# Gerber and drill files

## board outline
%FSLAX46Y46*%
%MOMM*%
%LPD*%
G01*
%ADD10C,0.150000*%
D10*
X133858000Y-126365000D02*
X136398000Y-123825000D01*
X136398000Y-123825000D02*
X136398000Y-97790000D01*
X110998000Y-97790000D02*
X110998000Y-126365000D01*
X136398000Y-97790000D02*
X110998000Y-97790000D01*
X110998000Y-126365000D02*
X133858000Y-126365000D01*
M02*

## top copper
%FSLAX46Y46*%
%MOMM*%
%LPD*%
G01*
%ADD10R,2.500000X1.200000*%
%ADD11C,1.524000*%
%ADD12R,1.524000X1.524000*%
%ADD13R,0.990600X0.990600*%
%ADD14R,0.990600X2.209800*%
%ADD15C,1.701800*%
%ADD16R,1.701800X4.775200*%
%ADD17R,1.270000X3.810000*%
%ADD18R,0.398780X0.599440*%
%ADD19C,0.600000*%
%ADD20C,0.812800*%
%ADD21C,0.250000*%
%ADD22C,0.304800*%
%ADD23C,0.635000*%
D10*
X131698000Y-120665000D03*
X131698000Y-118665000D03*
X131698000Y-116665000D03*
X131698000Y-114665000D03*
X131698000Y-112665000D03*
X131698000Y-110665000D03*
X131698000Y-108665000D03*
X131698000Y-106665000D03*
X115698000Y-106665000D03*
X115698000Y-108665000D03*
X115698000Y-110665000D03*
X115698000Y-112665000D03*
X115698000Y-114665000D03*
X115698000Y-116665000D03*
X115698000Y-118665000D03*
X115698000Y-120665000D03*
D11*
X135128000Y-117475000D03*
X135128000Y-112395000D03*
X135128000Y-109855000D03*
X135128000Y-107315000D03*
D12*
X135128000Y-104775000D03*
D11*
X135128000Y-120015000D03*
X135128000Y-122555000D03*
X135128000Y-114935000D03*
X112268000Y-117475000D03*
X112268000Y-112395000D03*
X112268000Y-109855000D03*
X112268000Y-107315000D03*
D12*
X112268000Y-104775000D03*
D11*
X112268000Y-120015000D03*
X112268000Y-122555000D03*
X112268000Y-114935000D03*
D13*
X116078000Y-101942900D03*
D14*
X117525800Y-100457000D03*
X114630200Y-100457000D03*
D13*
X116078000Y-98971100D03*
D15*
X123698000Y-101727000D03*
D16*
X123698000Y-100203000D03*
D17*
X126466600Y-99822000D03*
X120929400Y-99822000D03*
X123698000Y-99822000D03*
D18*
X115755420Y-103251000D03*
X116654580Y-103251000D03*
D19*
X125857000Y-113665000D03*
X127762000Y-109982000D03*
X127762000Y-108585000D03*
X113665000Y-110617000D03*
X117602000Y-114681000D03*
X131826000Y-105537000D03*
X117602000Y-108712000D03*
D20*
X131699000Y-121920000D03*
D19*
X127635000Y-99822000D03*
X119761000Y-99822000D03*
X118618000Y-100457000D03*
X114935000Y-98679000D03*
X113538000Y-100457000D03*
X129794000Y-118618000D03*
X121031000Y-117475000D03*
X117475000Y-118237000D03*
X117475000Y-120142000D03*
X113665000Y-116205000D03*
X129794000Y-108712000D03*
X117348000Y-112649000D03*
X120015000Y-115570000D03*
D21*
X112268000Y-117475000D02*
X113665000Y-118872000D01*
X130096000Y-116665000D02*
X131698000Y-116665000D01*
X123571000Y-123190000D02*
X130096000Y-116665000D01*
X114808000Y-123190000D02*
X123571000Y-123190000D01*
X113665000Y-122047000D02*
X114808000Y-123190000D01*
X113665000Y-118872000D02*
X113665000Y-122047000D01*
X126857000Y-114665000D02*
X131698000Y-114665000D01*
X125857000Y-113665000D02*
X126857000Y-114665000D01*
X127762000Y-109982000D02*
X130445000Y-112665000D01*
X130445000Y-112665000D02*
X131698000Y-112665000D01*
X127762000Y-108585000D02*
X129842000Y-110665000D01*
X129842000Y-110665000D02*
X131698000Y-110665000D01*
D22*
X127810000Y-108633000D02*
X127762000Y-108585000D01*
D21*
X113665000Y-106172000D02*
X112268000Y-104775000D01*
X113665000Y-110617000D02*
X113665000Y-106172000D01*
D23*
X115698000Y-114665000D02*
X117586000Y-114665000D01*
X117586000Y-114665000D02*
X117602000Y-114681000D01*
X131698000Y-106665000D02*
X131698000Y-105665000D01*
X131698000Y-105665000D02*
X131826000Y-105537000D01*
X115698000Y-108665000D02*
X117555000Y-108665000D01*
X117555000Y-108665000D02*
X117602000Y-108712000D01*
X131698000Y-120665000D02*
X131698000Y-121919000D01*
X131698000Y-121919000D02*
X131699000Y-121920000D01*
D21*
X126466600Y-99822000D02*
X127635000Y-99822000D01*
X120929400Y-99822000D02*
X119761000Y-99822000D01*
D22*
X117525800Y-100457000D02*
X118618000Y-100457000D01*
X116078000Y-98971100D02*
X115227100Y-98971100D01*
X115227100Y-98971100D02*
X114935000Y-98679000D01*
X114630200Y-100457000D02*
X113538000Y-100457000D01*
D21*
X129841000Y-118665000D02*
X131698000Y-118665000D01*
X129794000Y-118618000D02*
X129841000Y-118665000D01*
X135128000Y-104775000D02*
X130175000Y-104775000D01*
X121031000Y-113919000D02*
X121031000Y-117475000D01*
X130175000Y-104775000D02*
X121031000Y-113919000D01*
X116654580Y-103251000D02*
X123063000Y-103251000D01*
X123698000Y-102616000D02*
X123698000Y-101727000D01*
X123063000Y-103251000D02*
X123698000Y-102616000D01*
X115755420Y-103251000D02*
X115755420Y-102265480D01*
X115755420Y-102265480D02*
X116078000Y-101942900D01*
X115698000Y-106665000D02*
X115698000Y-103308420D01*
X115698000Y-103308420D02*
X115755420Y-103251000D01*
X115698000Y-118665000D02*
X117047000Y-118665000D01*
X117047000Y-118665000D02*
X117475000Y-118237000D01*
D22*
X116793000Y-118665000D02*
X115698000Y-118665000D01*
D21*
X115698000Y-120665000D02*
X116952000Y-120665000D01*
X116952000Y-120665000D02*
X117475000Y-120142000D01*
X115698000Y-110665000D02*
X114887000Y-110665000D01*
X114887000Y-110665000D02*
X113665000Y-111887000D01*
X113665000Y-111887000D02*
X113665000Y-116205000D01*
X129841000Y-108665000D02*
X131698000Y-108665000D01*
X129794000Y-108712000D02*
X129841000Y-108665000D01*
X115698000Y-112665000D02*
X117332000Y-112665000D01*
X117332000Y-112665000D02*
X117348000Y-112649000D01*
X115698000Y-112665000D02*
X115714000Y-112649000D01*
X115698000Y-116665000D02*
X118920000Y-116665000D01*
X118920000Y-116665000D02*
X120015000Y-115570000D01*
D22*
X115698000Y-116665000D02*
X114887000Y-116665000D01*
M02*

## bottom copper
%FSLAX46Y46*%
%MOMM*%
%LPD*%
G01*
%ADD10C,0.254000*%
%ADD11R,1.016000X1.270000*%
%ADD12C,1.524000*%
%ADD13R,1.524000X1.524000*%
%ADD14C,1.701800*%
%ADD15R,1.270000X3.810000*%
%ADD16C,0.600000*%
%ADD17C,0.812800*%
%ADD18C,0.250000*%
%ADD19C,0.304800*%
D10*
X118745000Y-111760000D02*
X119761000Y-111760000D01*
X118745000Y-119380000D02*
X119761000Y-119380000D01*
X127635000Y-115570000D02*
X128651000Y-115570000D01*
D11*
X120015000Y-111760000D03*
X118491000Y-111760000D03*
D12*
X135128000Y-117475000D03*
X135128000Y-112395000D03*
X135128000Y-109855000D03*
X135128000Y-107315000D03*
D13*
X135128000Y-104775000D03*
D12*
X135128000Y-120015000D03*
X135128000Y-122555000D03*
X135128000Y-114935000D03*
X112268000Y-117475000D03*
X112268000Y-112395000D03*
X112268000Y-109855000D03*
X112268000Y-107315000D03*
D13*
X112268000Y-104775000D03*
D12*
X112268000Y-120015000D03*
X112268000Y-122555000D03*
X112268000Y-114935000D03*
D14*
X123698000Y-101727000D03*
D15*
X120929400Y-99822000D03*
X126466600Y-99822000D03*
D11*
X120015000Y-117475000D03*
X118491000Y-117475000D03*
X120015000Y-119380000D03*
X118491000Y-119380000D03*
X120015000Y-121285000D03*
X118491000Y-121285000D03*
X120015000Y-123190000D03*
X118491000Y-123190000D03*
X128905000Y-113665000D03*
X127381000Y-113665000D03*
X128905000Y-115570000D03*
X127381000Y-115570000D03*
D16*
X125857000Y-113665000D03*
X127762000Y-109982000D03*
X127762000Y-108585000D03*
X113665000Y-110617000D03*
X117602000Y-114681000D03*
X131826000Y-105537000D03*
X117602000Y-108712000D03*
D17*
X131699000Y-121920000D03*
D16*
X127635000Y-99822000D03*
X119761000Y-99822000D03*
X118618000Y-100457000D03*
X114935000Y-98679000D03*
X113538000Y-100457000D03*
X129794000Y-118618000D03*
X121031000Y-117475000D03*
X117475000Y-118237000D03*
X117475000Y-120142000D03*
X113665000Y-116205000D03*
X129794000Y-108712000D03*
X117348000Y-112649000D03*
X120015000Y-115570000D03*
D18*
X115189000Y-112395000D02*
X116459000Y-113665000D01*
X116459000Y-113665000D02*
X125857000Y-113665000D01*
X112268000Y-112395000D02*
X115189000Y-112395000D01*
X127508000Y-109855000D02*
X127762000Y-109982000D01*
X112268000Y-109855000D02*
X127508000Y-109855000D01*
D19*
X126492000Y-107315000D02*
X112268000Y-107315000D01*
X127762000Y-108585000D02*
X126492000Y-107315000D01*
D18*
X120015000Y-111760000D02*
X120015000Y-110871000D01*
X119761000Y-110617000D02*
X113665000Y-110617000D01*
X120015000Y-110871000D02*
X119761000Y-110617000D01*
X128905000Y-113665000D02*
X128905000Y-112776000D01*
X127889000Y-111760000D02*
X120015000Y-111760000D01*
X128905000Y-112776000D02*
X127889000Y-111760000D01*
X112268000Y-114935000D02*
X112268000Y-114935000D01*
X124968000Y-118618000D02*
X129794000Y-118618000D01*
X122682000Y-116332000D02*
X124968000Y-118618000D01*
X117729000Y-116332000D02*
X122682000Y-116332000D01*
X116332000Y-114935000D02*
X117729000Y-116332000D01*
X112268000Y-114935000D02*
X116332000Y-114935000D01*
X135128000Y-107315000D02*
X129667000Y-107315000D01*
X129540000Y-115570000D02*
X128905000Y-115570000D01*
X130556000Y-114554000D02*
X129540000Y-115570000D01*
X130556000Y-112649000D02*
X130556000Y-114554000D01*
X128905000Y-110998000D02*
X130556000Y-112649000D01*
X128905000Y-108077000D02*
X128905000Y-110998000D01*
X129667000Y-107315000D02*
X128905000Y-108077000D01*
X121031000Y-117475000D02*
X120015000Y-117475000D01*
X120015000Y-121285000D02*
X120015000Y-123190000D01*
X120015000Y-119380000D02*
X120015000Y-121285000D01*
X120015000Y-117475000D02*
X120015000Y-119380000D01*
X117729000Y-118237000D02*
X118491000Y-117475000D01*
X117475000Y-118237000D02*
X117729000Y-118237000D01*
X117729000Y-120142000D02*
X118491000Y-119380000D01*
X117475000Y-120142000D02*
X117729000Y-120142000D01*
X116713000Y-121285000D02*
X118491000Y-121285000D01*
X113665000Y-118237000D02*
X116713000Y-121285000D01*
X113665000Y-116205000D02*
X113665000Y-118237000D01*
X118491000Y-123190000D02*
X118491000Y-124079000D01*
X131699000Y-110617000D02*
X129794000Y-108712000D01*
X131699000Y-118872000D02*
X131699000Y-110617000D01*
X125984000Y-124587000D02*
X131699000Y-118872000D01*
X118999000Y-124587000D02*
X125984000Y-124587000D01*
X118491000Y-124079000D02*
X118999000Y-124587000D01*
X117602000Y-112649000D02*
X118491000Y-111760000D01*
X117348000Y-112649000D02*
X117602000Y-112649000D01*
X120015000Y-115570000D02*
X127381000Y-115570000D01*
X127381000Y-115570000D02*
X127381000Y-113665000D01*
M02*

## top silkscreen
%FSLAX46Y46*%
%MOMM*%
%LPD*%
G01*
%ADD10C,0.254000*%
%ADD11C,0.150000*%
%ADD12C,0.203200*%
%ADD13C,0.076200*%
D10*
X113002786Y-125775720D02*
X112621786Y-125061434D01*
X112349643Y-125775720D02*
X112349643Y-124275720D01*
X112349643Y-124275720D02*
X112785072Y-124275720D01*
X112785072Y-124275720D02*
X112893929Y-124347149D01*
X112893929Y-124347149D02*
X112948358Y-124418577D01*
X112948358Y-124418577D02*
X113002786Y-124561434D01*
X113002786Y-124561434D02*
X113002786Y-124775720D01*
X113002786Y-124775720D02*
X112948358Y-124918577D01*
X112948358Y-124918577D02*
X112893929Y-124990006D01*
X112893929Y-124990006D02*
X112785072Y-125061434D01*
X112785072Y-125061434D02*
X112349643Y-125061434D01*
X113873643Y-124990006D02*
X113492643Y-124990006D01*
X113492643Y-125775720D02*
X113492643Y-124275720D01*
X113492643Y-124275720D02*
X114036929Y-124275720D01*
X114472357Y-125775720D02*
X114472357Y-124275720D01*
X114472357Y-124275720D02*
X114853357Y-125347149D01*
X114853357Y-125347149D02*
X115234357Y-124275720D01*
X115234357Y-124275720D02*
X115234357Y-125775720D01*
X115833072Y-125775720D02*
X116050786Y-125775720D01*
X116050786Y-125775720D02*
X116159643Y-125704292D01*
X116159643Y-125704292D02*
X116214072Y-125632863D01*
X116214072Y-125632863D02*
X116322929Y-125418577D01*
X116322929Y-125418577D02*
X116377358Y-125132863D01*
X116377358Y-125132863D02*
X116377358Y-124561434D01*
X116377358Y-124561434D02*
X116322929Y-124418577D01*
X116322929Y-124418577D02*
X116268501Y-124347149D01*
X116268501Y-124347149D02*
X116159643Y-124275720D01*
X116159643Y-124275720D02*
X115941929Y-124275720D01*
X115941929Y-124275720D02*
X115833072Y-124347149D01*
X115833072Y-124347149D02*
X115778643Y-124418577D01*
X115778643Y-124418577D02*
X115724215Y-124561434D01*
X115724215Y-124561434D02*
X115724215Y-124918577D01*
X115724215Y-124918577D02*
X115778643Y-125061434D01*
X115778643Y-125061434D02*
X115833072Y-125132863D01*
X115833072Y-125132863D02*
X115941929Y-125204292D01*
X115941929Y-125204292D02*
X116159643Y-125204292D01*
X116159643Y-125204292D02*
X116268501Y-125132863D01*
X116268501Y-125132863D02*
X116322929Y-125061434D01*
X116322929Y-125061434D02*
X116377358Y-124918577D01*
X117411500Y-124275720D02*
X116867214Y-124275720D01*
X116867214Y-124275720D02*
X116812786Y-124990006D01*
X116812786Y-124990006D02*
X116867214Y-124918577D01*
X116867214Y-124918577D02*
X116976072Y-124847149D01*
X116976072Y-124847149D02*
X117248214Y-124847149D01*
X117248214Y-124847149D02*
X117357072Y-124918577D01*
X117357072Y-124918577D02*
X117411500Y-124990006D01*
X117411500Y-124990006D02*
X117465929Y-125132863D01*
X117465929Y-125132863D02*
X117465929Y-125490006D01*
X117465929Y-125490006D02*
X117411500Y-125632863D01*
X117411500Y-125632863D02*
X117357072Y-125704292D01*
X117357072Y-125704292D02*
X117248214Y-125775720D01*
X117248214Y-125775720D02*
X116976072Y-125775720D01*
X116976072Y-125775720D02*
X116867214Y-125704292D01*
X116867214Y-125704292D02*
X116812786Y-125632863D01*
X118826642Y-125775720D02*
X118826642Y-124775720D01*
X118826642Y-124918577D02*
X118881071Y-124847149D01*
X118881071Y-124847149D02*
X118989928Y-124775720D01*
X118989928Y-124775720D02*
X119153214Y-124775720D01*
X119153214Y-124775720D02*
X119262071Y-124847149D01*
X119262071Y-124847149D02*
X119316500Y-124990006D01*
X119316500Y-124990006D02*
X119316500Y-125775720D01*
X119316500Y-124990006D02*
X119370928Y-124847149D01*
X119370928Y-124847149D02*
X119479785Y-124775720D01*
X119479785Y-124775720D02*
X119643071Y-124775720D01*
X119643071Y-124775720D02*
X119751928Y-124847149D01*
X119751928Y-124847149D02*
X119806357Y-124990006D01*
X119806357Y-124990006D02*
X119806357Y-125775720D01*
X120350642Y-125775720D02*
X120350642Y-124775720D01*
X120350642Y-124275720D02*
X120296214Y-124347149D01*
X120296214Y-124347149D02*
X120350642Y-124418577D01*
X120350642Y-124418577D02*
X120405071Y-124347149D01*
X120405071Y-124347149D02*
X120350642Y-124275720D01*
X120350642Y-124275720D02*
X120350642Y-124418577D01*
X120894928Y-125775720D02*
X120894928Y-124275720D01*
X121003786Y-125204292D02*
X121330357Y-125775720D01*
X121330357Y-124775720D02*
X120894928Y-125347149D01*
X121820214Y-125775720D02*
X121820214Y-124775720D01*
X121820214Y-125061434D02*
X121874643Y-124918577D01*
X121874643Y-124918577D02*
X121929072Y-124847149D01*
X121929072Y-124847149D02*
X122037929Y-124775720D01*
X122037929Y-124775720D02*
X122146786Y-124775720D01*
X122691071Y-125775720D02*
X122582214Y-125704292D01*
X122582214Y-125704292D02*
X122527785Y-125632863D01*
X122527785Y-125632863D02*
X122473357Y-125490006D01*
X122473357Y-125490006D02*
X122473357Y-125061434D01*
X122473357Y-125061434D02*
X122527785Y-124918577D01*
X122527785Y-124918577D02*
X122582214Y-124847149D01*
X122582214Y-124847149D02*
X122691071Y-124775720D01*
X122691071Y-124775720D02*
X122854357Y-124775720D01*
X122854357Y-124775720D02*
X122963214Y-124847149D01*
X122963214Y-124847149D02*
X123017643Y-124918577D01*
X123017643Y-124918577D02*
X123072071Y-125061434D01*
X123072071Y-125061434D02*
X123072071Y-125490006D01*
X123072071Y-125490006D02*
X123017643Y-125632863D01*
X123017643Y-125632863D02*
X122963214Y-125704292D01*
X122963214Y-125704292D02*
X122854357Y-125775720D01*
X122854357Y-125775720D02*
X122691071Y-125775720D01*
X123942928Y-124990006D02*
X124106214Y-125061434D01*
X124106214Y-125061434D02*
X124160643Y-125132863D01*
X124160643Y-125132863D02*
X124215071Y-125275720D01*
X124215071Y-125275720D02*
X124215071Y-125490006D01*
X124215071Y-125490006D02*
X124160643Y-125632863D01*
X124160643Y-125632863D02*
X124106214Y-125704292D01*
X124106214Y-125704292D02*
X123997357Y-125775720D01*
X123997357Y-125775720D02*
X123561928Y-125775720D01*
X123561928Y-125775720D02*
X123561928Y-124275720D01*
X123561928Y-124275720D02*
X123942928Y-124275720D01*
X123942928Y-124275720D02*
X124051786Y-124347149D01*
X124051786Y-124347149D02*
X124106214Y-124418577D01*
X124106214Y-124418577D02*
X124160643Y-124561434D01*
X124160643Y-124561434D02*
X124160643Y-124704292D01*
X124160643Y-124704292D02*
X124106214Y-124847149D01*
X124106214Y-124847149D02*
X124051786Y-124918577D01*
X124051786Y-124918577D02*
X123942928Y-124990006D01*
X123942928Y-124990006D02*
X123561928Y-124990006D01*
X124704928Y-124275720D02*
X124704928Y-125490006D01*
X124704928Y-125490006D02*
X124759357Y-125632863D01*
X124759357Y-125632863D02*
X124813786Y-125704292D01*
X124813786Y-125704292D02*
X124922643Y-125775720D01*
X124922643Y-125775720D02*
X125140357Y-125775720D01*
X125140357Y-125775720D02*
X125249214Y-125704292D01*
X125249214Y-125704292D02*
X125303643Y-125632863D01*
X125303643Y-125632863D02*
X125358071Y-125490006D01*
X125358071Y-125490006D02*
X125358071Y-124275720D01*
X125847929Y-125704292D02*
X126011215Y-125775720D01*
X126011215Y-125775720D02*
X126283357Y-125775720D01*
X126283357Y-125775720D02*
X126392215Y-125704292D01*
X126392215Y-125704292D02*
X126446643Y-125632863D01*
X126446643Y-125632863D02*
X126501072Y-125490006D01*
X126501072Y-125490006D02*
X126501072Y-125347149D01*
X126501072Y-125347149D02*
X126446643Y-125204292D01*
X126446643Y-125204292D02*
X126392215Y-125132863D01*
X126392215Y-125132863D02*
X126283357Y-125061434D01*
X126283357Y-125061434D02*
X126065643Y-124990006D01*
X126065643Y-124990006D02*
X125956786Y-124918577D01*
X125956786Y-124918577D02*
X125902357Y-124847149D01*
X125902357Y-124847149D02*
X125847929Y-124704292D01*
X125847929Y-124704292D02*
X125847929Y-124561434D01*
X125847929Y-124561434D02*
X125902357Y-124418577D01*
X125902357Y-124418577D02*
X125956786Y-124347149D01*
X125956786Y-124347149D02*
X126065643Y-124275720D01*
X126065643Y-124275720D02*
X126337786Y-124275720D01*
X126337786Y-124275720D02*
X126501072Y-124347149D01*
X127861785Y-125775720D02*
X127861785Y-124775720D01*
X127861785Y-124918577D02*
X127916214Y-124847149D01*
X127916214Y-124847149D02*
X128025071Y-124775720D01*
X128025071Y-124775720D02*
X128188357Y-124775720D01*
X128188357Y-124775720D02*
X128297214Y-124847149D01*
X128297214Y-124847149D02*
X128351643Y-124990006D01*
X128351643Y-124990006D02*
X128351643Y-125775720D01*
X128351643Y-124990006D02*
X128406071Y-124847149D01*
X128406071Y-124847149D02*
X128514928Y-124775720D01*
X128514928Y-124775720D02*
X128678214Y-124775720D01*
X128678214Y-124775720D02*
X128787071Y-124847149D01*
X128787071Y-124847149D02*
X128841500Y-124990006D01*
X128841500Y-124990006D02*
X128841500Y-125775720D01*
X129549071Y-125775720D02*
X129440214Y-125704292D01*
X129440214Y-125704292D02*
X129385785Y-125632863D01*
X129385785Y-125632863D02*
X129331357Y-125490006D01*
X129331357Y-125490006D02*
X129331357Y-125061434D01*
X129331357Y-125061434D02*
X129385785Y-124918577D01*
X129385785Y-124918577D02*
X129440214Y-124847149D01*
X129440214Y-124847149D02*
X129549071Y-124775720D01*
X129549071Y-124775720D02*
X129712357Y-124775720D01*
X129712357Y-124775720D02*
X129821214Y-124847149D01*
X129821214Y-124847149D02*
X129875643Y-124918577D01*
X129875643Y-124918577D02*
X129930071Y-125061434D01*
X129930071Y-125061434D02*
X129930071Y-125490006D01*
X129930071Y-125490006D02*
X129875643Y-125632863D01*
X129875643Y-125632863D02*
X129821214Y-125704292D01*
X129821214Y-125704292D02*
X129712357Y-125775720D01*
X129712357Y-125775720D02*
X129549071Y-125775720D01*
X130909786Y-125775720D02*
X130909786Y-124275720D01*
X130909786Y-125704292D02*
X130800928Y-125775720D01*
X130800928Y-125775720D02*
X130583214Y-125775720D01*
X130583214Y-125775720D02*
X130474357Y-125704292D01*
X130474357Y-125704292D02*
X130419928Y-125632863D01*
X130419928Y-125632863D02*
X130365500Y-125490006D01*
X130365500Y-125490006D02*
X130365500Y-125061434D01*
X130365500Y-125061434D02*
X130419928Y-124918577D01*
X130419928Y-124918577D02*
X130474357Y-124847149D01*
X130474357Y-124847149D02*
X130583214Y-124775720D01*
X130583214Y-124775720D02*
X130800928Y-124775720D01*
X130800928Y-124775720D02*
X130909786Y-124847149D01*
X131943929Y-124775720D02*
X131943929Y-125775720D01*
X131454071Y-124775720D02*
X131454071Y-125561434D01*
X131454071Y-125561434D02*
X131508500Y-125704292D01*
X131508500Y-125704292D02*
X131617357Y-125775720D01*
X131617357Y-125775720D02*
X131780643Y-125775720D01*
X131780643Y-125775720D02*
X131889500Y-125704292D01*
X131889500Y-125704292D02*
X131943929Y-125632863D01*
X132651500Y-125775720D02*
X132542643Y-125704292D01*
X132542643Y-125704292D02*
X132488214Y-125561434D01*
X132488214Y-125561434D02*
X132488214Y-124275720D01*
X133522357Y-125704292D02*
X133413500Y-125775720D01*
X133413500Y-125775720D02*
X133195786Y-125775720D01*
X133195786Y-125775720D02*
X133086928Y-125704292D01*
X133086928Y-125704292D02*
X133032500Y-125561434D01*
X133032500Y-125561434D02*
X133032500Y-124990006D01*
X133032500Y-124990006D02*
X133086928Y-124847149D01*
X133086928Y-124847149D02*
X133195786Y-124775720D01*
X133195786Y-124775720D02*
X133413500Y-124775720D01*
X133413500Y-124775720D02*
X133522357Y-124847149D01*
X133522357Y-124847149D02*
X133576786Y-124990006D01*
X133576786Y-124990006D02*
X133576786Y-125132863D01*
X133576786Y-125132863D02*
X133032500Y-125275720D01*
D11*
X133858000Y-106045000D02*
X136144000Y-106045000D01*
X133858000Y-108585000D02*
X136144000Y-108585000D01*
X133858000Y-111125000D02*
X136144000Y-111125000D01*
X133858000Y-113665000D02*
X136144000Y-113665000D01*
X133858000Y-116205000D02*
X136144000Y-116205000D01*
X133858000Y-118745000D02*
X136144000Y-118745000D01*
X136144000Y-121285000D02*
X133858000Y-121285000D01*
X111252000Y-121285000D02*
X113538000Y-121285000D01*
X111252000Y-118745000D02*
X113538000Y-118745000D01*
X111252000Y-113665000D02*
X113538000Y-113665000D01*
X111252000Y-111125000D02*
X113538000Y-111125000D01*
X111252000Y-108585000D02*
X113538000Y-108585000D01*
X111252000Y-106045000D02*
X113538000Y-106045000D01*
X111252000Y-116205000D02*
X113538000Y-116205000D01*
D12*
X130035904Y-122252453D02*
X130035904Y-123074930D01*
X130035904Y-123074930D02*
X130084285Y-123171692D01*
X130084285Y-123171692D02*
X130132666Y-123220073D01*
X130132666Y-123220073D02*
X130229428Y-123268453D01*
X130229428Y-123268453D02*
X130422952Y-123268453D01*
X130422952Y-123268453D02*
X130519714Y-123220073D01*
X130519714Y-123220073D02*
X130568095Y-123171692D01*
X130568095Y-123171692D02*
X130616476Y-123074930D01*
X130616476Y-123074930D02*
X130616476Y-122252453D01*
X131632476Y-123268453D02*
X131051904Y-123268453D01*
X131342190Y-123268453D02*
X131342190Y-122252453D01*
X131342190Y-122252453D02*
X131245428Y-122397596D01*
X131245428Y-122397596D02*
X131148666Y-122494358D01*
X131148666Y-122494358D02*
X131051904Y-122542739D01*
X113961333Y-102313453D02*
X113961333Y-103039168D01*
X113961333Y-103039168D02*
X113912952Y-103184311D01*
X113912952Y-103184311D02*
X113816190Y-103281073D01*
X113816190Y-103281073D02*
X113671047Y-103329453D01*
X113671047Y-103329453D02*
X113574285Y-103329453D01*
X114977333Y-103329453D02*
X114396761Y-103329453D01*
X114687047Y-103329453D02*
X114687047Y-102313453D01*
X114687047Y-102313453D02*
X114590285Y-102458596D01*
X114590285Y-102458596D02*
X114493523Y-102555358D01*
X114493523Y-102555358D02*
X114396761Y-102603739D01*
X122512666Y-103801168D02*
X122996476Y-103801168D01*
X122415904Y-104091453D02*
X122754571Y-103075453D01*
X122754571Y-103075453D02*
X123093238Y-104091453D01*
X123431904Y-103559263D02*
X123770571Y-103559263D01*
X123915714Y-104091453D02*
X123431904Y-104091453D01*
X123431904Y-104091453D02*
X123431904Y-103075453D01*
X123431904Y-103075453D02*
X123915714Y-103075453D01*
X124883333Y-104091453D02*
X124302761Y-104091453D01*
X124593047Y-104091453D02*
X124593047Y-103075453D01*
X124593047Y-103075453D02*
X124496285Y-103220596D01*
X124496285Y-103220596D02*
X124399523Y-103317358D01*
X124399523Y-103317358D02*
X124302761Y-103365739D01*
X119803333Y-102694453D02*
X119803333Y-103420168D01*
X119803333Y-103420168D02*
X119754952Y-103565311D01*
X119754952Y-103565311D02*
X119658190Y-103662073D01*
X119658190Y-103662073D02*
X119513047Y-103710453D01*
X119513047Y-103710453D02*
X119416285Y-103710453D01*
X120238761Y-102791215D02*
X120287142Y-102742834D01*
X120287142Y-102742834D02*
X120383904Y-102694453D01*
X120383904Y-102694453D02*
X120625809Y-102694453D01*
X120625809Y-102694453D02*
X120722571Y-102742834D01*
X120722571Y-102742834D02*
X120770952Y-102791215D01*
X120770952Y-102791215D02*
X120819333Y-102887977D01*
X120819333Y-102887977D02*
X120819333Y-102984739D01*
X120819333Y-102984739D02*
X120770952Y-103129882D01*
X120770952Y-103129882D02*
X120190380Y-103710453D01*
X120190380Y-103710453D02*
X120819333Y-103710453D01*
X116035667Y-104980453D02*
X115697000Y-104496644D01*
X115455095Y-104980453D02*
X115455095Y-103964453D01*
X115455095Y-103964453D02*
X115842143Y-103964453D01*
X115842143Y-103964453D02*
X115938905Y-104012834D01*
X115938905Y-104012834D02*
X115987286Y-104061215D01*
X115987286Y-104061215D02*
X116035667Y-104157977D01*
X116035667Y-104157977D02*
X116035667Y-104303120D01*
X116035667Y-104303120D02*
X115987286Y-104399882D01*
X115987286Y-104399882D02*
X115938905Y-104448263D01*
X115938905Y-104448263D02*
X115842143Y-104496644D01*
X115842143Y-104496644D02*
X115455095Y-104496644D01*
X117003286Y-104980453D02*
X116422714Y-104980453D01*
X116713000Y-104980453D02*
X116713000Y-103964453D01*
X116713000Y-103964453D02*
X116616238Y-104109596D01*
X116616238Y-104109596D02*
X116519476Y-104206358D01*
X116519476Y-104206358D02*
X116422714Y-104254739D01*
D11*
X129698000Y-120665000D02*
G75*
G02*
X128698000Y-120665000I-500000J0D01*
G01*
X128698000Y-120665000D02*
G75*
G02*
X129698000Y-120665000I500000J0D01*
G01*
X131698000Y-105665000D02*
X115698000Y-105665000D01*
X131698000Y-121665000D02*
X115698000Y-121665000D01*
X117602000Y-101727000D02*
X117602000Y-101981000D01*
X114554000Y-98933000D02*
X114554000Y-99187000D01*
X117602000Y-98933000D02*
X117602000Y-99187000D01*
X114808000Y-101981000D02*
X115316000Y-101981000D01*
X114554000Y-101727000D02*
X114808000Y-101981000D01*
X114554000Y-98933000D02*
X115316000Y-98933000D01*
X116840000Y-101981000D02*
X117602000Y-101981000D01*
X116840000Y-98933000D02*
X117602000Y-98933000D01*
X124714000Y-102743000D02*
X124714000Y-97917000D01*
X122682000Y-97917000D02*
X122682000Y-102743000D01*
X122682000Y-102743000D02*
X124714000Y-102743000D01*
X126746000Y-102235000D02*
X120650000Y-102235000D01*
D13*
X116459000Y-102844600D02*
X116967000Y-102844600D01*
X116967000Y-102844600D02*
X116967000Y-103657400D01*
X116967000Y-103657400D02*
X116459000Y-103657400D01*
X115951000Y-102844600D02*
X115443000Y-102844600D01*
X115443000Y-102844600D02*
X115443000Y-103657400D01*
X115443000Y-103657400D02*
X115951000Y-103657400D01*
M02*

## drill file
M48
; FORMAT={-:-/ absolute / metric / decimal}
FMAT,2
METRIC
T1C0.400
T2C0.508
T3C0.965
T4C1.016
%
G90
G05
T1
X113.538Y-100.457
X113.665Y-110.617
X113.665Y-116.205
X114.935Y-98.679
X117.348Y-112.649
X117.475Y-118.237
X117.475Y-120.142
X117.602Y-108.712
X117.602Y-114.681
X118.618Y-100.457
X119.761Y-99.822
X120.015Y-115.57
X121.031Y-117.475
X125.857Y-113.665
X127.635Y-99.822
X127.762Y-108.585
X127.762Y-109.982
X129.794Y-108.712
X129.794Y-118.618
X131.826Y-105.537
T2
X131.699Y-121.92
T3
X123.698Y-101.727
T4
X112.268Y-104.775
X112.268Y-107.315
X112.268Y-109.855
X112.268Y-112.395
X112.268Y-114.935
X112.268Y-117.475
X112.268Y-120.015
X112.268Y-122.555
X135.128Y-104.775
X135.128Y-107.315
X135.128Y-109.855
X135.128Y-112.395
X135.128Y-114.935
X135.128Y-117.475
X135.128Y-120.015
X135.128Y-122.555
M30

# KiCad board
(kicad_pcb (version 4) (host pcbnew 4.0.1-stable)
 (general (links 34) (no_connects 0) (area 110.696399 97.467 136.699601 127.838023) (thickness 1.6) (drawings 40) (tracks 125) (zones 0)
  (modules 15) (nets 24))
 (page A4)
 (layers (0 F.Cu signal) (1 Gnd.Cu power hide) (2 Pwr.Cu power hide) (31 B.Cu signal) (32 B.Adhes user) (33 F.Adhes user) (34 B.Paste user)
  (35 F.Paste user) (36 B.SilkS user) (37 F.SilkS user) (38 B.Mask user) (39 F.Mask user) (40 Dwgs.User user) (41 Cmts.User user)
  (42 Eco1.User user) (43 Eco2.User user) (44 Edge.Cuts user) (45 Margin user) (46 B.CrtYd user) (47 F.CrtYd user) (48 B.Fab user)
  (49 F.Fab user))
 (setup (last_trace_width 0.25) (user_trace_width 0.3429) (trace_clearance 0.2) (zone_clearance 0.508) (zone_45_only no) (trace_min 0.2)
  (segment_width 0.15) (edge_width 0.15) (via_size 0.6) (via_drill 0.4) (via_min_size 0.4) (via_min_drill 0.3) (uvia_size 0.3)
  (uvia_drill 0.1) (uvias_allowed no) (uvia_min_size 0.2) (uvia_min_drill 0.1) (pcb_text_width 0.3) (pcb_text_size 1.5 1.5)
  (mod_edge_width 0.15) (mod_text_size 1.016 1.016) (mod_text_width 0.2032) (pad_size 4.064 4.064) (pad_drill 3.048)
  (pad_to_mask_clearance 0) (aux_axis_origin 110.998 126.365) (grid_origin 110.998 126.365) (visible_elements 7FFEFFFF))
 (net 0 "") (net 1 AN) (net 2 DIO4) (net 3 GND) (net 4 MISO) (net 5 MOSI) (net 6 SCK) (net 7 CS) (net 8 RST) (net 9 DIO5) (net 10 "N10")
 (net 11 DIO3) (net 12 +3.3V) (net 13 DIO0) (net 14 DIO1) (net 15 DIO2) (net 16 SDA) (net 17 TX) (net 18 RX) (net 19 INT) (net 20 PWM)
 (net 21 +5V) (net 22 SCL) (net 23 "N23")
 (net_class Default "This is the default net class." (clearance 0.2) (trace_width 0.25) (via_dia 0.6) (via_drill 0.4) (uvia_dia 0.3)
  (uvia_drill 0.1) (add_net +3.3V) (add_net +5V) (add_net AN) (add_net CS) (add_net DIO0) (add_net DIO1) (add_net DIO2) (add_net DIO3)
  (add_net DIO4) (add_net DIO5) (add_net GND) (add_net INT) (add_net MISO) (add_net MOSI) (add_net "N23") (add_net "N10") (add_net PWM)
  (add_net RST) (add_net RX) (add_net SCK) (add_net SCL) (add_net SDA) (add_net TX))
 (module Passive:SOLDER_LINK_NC (layer B.Cu) (at 119.253 111.76 90)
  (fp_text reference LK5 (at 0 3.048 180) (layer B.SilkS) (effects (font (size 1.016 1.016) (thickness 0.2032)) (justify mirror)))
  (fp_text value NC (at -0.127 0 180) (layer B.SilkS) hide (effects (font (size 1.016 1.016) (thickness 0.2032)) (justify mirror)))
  (fp_line (start 0 -0.508) (end 0 0.508) (layer B.Cu) (width 0.254))
  (pad 1 smd rect (at 0 0.762 90) (size 1.27 1.016) (layers B.Cu B.Paste B.Mask) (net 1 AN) (solder_mask_margin 0.3048))
  (pad 2 smd rect (at 0 -0.762 90) (size 1.27 1.016) (layers B.Cu B.Paste B.Mask) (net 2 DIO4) (solder_mask_margin 0.3048)))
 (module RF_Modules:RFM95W (layer F.Cu) (at 123.698 113.665 180)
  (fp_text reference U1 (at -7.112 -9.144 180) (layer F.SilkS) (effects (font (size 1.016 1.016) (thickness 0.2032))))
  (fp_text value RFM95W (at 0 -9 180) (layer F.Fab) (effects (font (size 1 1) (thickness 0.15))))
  (fp_circle (center -5.5 -7) (end -5.5 -6.5) (layer F.SilkS) (width 0.15))
  (fp_line (start -8 8) (end 8 8) (layer F.SilkS) (width 0.15))
  (fp_line (start -8 -8) (end 8 -8) (layer F.SilkS) (width 0.15))
  (pad 1 smd rect (at -8 -7 180) (size 2.5 1.2) (layers F.Cu F.Paste F.Mask) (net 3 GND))
  (pad 2 smd rect (at -8 -5 180) (size 2.5 1.2) (layers F.Cu F.Paste F.Mask) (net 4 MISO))
  (pad 3 smd rect (at -8 -3 180) (size 2.5 1.2) (layers F.Cu F.Paste F.Mask) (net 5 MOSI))
  (pad 4 smd rect (at -8 -1 180) (size 2.5 1.2) (layers F.Cu F.Paste F.Mask) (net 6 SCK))
  (pad 5 smd rect (at -8 1 180) (size 2.5 1.2) (layers F.Cu F.Paste F.Mask) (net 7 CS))
  (pad 6 smd rect (at -8 3 180) (size 2.5 1.2) (layers F.Cu F.Paste F.Mask) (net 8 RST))
  (pad 7 smd rect (at -8 5 180) (size 2.5 1.2) (layers F.Cu F.Paste F.Mask) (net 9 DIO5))
  (pad 8 smd rect (at -8 7 180) (size 2.5 1.2) (layers F.Cu F.Paste F.Mask) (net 3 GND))
  (pad 9 smd rect (at 8 7 180) (size 2.5 1.2) (layers F.Cu F.Paste F.Mask) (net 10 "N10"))
  (pad 10 smd rect (at 8 5 180) (size 2.5 1.2) (layers F.Cu F.Paste F.Mask) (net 3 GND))
  (pad 11 smd rect (at 8 3 180) (size 2.5 1.2) (layers F.Cu F.Paste F.Mask) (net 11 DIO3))
  (pad 12 smd rect (at 8 1 180) (size 2.5 1.2) (layers F.Cu F.Paste F.Mask) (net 2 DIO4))
  (pad 13 smd rect (at 8 -1 180) (size 2.5 1.2) (layers F.Cu F.Paste F.Mask) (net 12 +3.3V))
  (pad 14 smd rect (at 8 -3 180) (size 2.5 1.2) (layers F.Cu F.Paste F.Mask) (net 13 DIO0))
  (pad 15 smd rect (at 8 -5 180) (size 2.5 1.2) (layers F.Cu F.Paste F.Mask) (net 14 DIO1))
  (pad 16 smd rect (at 8 -7 180) (size 2.5 1.2) (layers F.Cu F.Paste F.Mask) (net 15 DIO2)))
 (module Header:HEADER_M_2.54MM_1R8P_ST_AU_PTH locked (layer B.Cu) (at 135.128 113.665 270)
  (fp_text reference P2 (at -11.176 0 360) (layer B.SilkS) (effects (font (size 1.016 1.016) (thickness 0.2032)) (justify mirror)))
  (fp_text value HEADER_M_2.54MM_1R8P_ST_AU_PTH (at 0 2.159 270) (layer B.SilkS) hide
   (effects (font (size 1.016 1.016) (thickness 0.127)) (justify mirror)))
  (pad 6 thru_hole circle (at 3.81 0 270) (size 1.524 1.524) (drill 1.016) (layers *.Cu *.Mask) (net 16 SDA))
  (pad 4 thru_hole circle (at -1.27 0 270) (size 1.524 1.524) (drill 1.016) (layers *.Cu *.Mask) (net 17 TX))
  (pad 3 thru_hole circle (at -3.81 0 270) (size 1.524 1.524) (drill 1.016) (layers *.Cu *.Mask) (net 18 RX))
  (pad 2 thru_hole circle (at -6.35 0 270) (size 1.524 1.524) (drill 1.016) (layers *.Cu *.Mask) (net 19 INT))
  (pad 1 thru_hole rect (at -8.89 0 270) (size 1.524 1.524) (drill 1.016) (layers *.Cu *.Mask) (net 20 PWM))
  (pad 7 thru_hole circle (at 6.35 0 270) (size 1.524 1.524) (drill 1.016) (layers *.Cu *.Mask) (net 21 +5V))
  (pad 8 thru_hole circle (at 8.89 0 270) (size 1.524 1.524) (drill 1.016) (layers *.Cu *.Mask) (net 3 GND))
  (pad 5 thru_hole circle (at 1.27 0 270) (size 1.524 1.524) (drill 1.016) (layers *.Cu *.Mask) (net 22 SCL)))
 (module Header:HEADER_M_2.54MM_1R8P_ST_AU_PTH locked (layer B.Cu) (at 112.268 113.665 270)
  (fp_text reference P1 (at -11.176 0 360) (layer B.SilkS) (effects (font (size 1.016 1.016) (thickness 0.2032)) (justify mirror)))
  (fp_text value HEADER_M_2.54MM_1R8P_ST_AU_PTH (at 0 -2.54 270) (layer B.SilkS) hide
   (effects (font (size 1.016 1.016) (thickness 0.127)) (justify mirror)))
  (pad 6 thru_hole circle (at 3.81 0 270) (size 1.524 1.524) (drill 1.016) (layers *.Cu *.Mask) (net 5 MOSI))
  (pad 4 thru_hole circle (at -1.27 0 270) (size 1.524 1.524) (drill 1.016) (layers *.Cu *.Mask) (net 6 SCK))
  (pad 3 thru_hole circle (at -3.81 0 270) (size 1.524 1.524) (drill 1.016) (layers *.Cu *.Mask) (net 7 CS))
  (pad 2 thru_hole circle (at -6.35 0 270) (size 1.524 1.524) (drill 1.016) (layers *.Cu *.Mask) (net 8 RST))
  (pad 1 thru_hole rect (at -8.89 0 270) (size 1.524 1.524) (drill 1.016) (layers *.Cu *.Mask) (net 1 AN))
  (pad 7 thru_hole circle (at 6.35 0 270) (size 1.524 1.524) (drill 1.016) (layers *.Cu *.Mask) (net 12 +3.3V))
  (pad 8 thru_hole circle (at 8.89 0 270) (size 1.524 1.524) (drill 1.016) (layers *.Cu *.Mask) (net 3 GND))
  (pad 5 thru_hole circle (at 1.27 0 270) (size 1.524 1.524) (drill 1.016) (layers *.Cu *.Mask) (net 4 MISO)))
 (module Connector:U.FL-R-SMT (layer F.Cu) (at 116.078 100.457)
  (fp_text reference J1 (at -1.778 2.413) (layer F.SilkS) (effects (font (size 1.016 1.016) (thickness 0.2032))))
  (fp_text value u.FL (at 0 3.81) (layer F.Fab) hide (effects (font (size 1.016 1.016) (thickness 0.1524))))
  (fp_line (start 1.524 1.27) (end 1.524 1.524) (layer F.SilkS) (width 0.15))
  (fp_line (start -1.524 -1.524) (end -1.524 -1.27) (layer F.SilkS) (width 0.15))
  (fp_line (start 1.524 -1.524) (end 1.524 -1.27) (layer F.SilkS) (width 0.15))
  (fp_line (start -1.27 1.524) (end -0.762 1.524) (layer F.SilkS) (width 0.15))
  (fp_line (start -1.524 1.27) (end -1.27 1.524) (layer F.SilkS) (width 0.15))
  (fp_line (start -1.524 -1.524) (end -0.762 -1.524) (layer F.SilkS) (width 0.15))
  (fp_line (start 0.762 1.524) (end 1.524 1.524) (layer F.SilkS) (width 0.15))
  (fp_line (start 0.762 -1.524) (end 1.524 -1.524) (layer F.SilkS) (width 0.15))
  (pad 1 smd rect (at 0 1.4859) (size 0.9906 0.9906) (layers F.Cu F.Paste F.Mask) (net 10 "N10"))
  (pad 4 smd rect (at 1.4478 0) (size 0.9906 2.2098) (layers F.Cu F.Paste F.Mask) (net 3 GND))
  (pad 2 smd rect (at -1.4478 0) (size 0.9906 2.2098) (layers F.Cu F.Paste F.Mask) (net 3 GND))
  (pad 3 smd rect (at 0 -1.4859) (size 0.9906 0.9906) (layers F.Cu F.Paste F.Mask) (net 3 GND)))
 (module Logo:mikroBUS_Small (layer B.Cu) (at 123.698 104.775 180)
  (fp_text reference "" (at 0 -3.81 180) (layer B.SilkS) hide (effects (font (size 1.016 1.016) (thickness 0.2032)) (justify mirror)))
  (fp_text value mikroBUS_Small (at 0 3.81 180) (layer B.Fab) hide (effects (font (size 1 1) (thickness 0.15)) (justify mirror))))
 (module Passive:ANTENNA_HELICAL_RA (layer F.Cu) (at 123.698 101.727)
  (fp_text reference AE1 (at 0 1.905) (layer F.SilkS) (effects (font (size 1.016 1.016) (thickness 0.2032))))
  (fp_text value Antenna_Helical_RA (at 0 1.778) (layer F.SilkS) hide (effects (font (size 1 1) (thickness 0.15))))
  (fp_line (start 1.016 1.016) (end 1.016 -3.81) (layer F.SilkS) (width 0.15))
  (fp_line (start -1.016 -3.81) (end -1.016 1.016) (layer F.SilkS) (width 0.15))
  (fp_line (start -1.016 1.016) (end 1.016 1.016) (layer F.SilkS) (width 0.15))
  (pad 1 thru_hole circle (at 0 0) (size 1.7018 1.7018) (drill 0.9652) (layers *.Cu *.Mask) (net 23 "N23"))
  (pad 1 smd rect (at 0 -1.524) (size 1.7018 4.7752) (layers F.Cu F.Mask) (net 23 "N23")))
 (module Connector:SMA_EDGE (layer F.Cu) (at 123.698 97.917 270)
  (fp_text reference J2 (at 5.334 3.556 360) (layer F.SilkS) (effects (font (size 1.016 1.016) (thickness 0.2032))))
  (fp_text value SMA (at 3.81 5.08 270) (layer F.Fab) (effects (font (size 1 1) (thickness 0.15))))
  (fp_line (start 4.318 -3.048) (end 4.318 3.048) (layer F.SilkS) (width 0.15))
  (pad "" smd rect (at 1.905 2.7686 270) (size 3.81 1.27) (layers B.Cu))
  (pad "" smd rect (at 1.905 -2.7686 270) (size 3.81 1.27) (layers B.Cu))
  (pad 2 smd rect (at 1.905 -2.7686 270) (size 3.81 1.27) (layers F.Cu) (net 3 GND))
  (pad 3 smd rect (at 1.905 2.7686 270) (size 3.81 1.27) (layers F.Cu) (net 3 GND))
  (pad 1 smd rect (at 1.905 0 270) (size 3.81 1.27) (layers F.Cu F.Paste F.Mask) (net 23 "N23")))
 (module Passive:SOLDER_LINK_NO (layer B.Cu) (at 119.253 117.475 90)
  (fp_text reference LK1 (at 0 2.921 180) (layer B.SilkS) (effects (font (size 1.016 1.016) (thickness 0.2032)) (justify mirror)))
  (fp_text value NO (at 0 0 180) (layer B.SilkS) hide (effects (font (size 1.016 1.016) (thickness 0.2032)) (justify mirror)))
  (pad 1 smd rect (at 0 0.762 90) (size 1.27 1.016) (layers B.Cu B.Paste B.Mask) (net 20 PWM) (solder_mask_margin 0.3048))
  (pad 2 smd rect (at 0 -0.762 90) (size 1.27 1.016) (layers B.Cu B.Paste B.Mask) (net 14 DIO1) (solder_mask_margin 0.3048)))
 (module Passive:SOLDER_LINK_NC (layer B.Cu) (at 119.253 119.38 90)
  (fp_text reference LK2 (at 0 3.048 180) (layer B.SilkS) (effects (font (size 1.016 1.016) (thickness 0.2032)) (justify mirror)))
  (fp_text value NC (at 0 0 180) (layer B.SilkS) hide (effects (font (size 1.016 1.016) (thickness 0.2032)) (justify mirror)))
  (fp_line (start 0 -0.508) (end 0 0.508) (layer B.Cu) (width 0.254))
  (pad 1 smd rect (at 0 0.762 90) (size 1.27 1.016) (layers B.Cu B.Paste B.Mask) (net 20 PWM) (solder_mask_margin 0.3048))
  (pad 2 smd rect (at 0 -0.762 90) (size 1.27 1.016) (layers B.Cu B.Paste B.Mask) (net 15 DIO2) (solder_mask_margin 0.3048)))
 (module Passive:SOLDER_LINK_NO (layer B.Cu) (at 119.253 121.285 90)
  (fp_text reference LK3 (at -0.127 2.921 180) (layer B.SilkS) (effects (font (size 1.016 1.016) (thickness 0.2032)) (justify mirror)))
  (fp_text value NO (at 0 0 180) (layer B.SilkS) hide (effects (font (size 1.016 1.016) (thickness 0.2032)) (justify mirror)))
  (pad 1 smd rect (at 0 0.762 90) (size 1.27 1.016) (layers B.Cu B.Paste B.Mask) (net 20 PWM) (solder_mask_margin 0.3048))
  (pad 2 smd rect (at 0 -0.762 90) (size 1.27 1.016) (layers B.Cu B.Paste B.Mask) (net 11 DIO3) (solder_mask_margin 0.3048)))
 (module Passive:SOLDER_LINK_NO (layer B.Cu) (at 119.253 123.19 90)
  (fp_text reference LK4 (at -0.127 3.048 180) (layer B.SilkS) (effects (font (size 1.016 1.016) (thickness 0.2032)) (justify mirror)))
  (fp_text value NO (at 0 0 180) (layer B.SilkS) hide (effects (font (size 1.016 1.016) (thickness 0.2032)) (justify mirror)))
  (pad 1 smd rect (at 0 0.762 90) (size 1.27 1.016) (layers B.Cu B.Paste B.Mask) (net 20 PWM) (solder_mask_margin 0.3048))
  (pad 2 smd rect (at 0 -0.762 90) (size 1.27 1.016) (layers B.Cu B.Paste B.Mask) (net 9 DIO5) (solder_mask_margin 0.3048)))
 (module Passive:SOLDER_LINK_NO (layer B.Cu) (at 128.143 113.665 90)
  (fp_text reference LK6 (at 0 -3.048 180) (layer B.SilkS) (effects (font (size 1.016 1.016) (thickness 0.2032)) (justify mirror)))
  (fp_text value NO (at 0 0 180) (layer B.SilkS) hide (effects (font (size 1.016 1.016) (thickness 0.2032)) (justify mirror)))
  (pad 1 smd rect (at 0 0.762 90) (size 1.27 1.016) (layers B.Cu B.Paste B.Mask) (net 1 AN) (solder_mask_margin 0.3048))
  (pad 2 smd rect (at 0 -0.762 90) (size 1.27 1.016) (layers B.Cu B.Paste B.Mask) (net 13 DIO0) (solder_mask_margin 0.3048)))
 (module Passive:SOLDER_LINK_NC (layer B.Cu) (at 128.143 115.57 90)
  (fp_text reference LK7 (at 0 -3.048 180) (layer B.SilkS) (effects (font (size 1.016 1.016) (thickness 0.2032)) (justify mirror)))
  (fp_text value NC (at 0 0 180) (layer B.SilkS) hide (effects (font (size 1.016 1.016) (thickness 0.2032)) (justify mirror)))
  (fp_line (start 0 -0.508) (end 0 0.508) (layer B.Cu) (width 0.254))
  (pad 1 smd rect (at 0 0.762 90) (size 1.27 1.016) (layers B.Cu B.Paste B.Mask) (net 19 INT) (solder_mask_margin 0.3048))
  (pad 2 smd rect (at 0 -0.762 90) (size 1.27 1.016) (layers B.Cu B.Paste B.Mask) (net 13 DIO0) (solder_mask_margin 0.3048)))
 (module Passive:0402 (layer F.Cu) (at 116.205 103.251)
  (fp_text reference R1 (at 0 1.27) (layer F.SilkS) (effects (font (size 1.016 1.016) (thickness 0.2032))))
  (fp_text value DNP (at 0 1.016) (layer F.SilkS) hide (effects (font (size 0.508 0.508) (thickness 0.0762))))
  (fp_line (start 0.254 -0.4064) (end 0.762 -0.4064) (layer F.SilkS) (width 0.0762))
  (fp_line (start 0.762 -0.4064) (end 0.762 0.4064) (layer F.SilkS) (width 0.0762))
  (fp_line (start 0.762 0.4064) (end 0.254 0.4064) (layer F.SilkS) (width 0.0762))
  (fp_line (start -0.254 -0.4064) (end -0.762 -0.4064) (layer F.SilkS) (width 0.0762))
  (fp_line (start -0.762 -0.4064) (end -0.762 0.4064) (layer F.SilkS) (width 0.0762))
  (fp_line (start -0.762 0.4064) (end -0.254 0.4064) (layer F.SilkS) (width 0.0762))
  (pad 1 smd rect (at -0.44958 0) (size 0.39878 0.59944) (layers F.Cu F.Paste F.Mask) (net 10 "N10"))
  (pad 2 smd rect (at 0.44958 0) (size 0.39878 0.59944) (layers F.Cu F.Paste F.Mask) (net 23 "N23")))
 (gr_line (start 133.858 126.365) (end 136.398 123.825) (angle 90) (layer Edge.Cuts) (width 0.15))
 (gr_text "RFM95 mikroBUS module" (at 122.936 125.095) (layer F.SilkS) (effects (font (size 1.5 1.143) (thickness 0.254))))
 (gr_line (start 136.398 123.825) (end 136.398 97.79) (angle 90) (layer Edge.Cuts) (width 0.15))
 (gr_line (start 110.998 97.79) (end 110.998 126.365) (angle 90) (layer Edge.Cuts) (width 0.15))
 (gr_line (start 136.398 97.79) (end 110.998 97.79) (angle 90) (layer Edge.Cuts) (width 0.15))
 (gr_line (start 110.998 126.365) (end 133.858 126.365) (angle 90) (layer Edge.Cuts) (width 0.15))
 (gr_line (start 133.858 106.045) (end 136.144 106.045) (angle 90) (layer F.SilkS) (width 0.15))
 (gr_line (start 133.858 108.585) (end 136.144 108.585) (angle 90) (layer F.SilkS) (width 0.15))
 (gr_line (start 133.858 111.125) (end 136.144 111.125) (angle 90) (layer F.SilkS) (width 0.15))
 (gr_line (start 133.858 113.665) (end 136.144 113.665) (angle 90) (layer F.SilkS) (width 0.15))
 (gr_line (start 133.858 116.205) (end 136.144 116.205) (angle 90) (layer F.SilkS) (width 0.15))
 (gr_line (start 133.858 118.745) (end 136.144 118.745) (angle 90) (layer F.SilkS) (width 0.15))
 (gr_line (start 136.144 121.285) (end 133.858 121.285) (angle 90) (layer F.SilkS) (width 0.15))
 (gr_line (start 111.252 121.285) (end 113.538 121.285) (angle 90) (layer F.SilkS) (width 0.15))
 (gr_line (start 111.252 118.745) (end 113.538 118.745) (angle 90) (layer F.SilkS) (width 0.15))
 (gr_line (start 111.252 113.665) (end 113.538 113.665) (angle 90) (layer F.SilkS) (width 0.15))
 (gr_line (start 111.252 111.125) (end 113.538 111.125) (angle 90) (layer F.SilkS) (width 0.15))
 (gr_line (start 111.252 108.585) (end 113.538 108.585) (angle 90) (layer F.SilkS) (width 0.15))
 (gr_line (start 111.252 106.045) (end 113.538 106.045) (angle 90) (layer F.SilkS) (width 0.15))
 (gr_line (start 111.252 116.205) (end 113.538 116.205) (angle 90) (layer F.SilkS) (width 0.15))
 (segment (start 112.268 117.475) (end 113.665 118.872) (width 0.25) (layer F.Cu) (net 5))
 (segment (start 130.096 116.665) (end 131.698 116.665) (width 0.25) (layer F.Cu) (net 5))
 (segment (start 123.571 123.19) (end 130.096 116.665) (width 0.25) (layer F.Cu) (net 5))
 (segment (start 114.808 123.19) (end 123.571 123.19) (width 0.25) (layer F.Cu) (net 5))
 (segment (start 113.665 122.047) (end 114.808 123.19) (width 0.25) (layer F.Cu) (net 5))
 (segment (start 113.665 118.872) (end 113.665 122.047) (width 0.25) (layer F.Cu) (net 5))
 (via (at 125.857 113.665) (size 0.6) (drill 0.4) (layers F.Cu B.Cu) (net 6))
 (segment (start 115.189 112.395) (end 116.459 113.665) (width 0.25) (layer B.Cu) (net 6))
 (segment (start 116.459 113.665) (end 125.857 113.665) (width 0.25) (layer B.Cu) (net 6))
 (segment (start 112.268 112.395) (end 115.189 112.395) (width 0.25) (layer B.Cu) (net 6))
 (segment (start 126.857 114.665) (end 131.698 114.665) (width 0.25) (layer F.Cu) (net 6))
 (segment (start 125.857 113.665) (end 126.857 114.665) (width 0.25) (layer F.Cu) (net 6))
 (segment (start 127.762 109.982) (end 130.445 112.665) (width 0.25) (layer F.Cu) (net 7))
 (segment (start 127.508 109.855) (end 127.762 109.982) (width 0.25) (layer B.Cu) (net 7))
 (via (at 127.762 109.982) (size 0.6) (drill 0.4) (layers F.Cu B.Cu) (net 7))
 (segment (start 112.268 109.855) (end 127.508 109.855) (width 0.25) (layer B.Cu) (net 7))
 (segment (start 130.445 112.665) (end 131.698 112.665) (width 0.25) (layer F.Cu) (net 7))
 (segment (start 127.762 108.585) (end 129.842 110.665) (width 0.25) (layer F.Cu) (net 8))
 (segment (start 129.842 110.665) (end 131.698 110.665) (width 0.25) (layer F.Cu) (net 8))
 (segment (start 126.492 107.315) (end 112.268 107.315) (width 0.3048) (layer B.Cu) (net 8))
 (segment (start 127.762 108.585) (end 126.492 107.315) (width 0.3048) (layer B.Cu) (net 8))
 (via (at 127.762 108.585) (size 0.6) (drill 0.4) (layers F.Cu B.Cu) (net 8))
 (segment (start 127.81 108.633) (end 127.762 108.585) (width 0.3048) (layer F.Cu) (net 8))
 (segment (start 120.015 111.76) (end 120.015 110.871) (width 0.25) (layer B.Cu) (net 1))
 (segment (start 113.665 106.172) (end 112.268 104.775) (width 0.25) (layer F.Cu) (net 1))
 (segment (start 113.665 110.617) (end 113.665 106.172) (width 0.25) (layer F.Cu) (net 1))
 (via (at 113.665 110.617) (size 0.6) (drill 0.4) (layers F.Cu B.Cu) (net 1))
 (segment (start 119.761 110.617) (end 113.665 110.617) (width 0.25) (layer B.Cu) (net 1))
 (segment (start 120.015 110.871) (end 119.761 110.617) (width 0.25) (layer B.Cu) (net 1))
 (segment (start 128.905 113.665) (end 128.905 112.776) (width 0.25) (layer B.Cu) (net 1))
 (segment (start 127.889 111.76) (end 120.015 111.76) (width 0.25) (layer B.Cu) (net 1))
 (segment (start 128.905 112.776) (end 127.889 111.76) (width 0.25) (layer B.Cu) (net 1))
 (segment (start 115.698 114.665) (end 117.586 114.665) (width 0.635) (layer F.Cu) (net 12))
 (via (at 117.602 114.681) (size 0.6) (drill 0.4) (layers F.Cu B.Cu) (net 12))
 (segment (start 117.586 114.665) (end 117.602 114.681) (width 0.635) (layer F.Cu) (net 12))
 (segment (start 131.698 106.665) (end 131.698 105.665) (width 0.635) (layer F.Cu) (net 3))
 (via (at 131.826 105.537) (size 0.6) (drill 0.4) (layers F.Cu B.Cu) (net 3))
 (segment (start 131.698 105.665) (end 131.826 105.537) (width 0.635) (layer F.Cu) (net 3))
 (segment (start 115.698 108.665) (end 117.555 108.665) (width 0.635) (layer F.Cu) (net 3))
 (via (at 117.602 108.712) (size 0.6) (drill 0.4) (layers F.Cu B.Cu) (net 3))
 (segment (start 117.555 108.665) (end 117.602 108.712) (width 0.635) (layer F.Cu) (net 3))
 (segment (start 131.698 120.665) (end 131.698 121.919) (width 0.635) (layer F.Cu) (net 3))
 (via (at 131.699 121.92) (size 0.8128) (drill 0.508) (layers F.Cu B.Cu) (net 3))
 (segment (start 131.698 121.919) (end 131.699 121.92) (width 0.635) (layer F.Cu) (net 3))
 (segment (start 126.4666 99.822) (end 127.635 99.822) (width 0.25) (layer F.Cu) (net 3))
 (via (at 127.635 99.822) (size 0.6) (drill 0.4) (layers F.Cu B.Cu) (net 3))
 (segment (start 120.9294 99.822) (end 119.761 99.822) (width 0.25) (layer F.Cu) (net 3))
 (via (at 119.761 99.822) (size 0.6) (drill 0.4) (layers F.Cu B.Cu) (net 3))
 (segment (start 117.5258 100.457) (end 118.618 100.457) (width 0.3048) (layer F.Cu) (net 3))
 (via (at 118.618 100.457) (size 0.6) (drill 0.4) (layers F.Cu B.Cu) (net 3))
 (segment (start 116.078 98.9711) (end 115.2271 98.9711) (width 0.3048) (layer F.Cu) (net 3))
 (via (at 114.935 98.679) (size 0.6) (drill 0.4) (layers F.Cu B.Cu) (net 3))
 (segment (start 115.2271 98.9711) (end 114.935 98.679) (width 0.3048) (layer F.Cu) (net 3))
 (segment (start 114.6302 100.457) (end 113.538 100.457) (width 0.3048) (layer F.Cu) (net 3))
 (via (at 113.538 100.457) (size 0.6) (drill 0.4) (layers F.Cu B.Cu) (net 3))
 (segment (start 112.268 114.935) (end 112.268 114.935) (width 0.25) (layer B.Cu) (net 4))
 (segment (start 129.841 118.665) (end 131.698 118.665) (width 0.25) (layer F.Cu) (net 4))
 (segment (start 129.794 118.618) (end 129.841 118.665) (width 0.25) (layer F.Cu) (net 4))
 (via (at 129.794 118.618) (size 0.6) (drill 0.4) (layers F.Cu B.Cu) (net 4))
 (segment (start 124.968 118.618) (end 129.794 118.618) (width 0.25) (layer B.Cu) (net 4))
 (segment (start 122.682 116.332) (end 124.968 118.618) (width 0.25) (layer B.Cu) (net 4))
 (segment (start 117.729 116.332) (end 122.682 116.332) (width 0.25) (layer B.Cu) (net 4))
 (segment (start 116.332 114.935) (end 117.729 116.332) (width 0.25) (layer B.Cu) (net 4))
 (segment (start 112.268 114.935) (end 116.332 114.935) (width 0.25) (layer B.Cu) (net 4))
 (segment (start 135.128 107.315) (end 129.667 107.315) (width 0.25) (layer B.Cu) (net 19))
 (segment (start 129.54 115.57) (end 128.905 115.57) (width 0.25) (layer B.Cu) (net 19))
 (segment (start 130.556 114.554) (end 129.54 115.57) (width 0.25) (layer B.Cu) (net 19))
 (segment (start 130.556 112.649) (end 130.556 114.554) (width 0.25) (layer B.Cu) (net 19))
 (segment (start 128.905 110.998) (end 130.556 112.649) (width 0.25) (layer B.Cu) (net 19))
 (segment (start 128.905 108.077) (end 128.905 110.998) (width 0.25) (layer B.Cu) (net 19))
 (segment (start 129.667 107.315) (end 128.905 108.077) (width 0.25) (layer B.Cu) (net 19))
 (segment (start 135.128 104.775) (end 130.175 104.775) (width 0.25) (layer F.Cu) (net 20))
 (segment (start 121.031 117.475) (end 120.015 117.475) (width 0.25) (layer B.Cu) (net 20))
 (via (at 121.031 117.475) (size 0.6) (drill 0.4) (layers F.Cu B.Cu) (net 20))
 (segment (start 121.031 113.919) (end 121.031 117.475) (width 0.25) (layer F.Cu) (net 20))
 (segment (start 130.175 104.775) (end 121.031 113.919) (width 0.25) (layer F.Cu) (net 20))
 (segment (start 120.015 121.285) (end 120.015 123.19) (width 0.25) (layer B.Cu) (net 20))
 (segment (start 120.015 119.38) (end 120.015 121.285) (width 0.25) (layer B.Cu) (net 20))
 (segment (start 120.015 117.475) (end 120.015 119.38) (width 0.25) (layer B.Cu) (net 20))
 (segment (start 116.65458 103.251) (end 123.063 103.251) (width 0.25) (layer F.Cu) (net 23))
 (segment (start 123.698 102.616) (end 123.698 101.727) (width 0.25) (layer F.Cu) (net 23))
 (segment (start 123.063 103.251) (end 123.698 102.616) (width 0.25) (layer F.Cu) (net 23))
 (segment (start 115.75542 103.251) (end 115.75542 102.26548) (width 0.25) (layer F.Cu) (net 10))
 (segment (start 115.75542 102.26548) (end 116.078 101.9429) (width 0.25) (layer F.Cu) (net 10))
 (segment (start 115.698 106.665) (end 115.698 103.30842) (width 0.25) (layer F.Cu) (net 10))
 (segment (start 115.698 103.30842) (end 115.75542 103.251) (width 0.25) (layer F.Cu) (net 10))
 (segment (start 115.698 118.665) (end 117.047 118.665) (width 0.25) (layer F.Cu) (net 14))
 (segment (start 117.729 118.237) (end 118.491 117.475) (width 0.25) (layer B.Cu) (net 14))
 (segment (start 117.475 118.237) (end 117.729 118.237) (width 0.25) (layer B.Cu) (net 14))
 (via (at 117.475 118.237) (size 0.6) (drill 0.4) (layers F.Cu B.Cu) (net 14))
 (segment (start 117.047 118.665) (end 117.475 118.237) (width 0.25) (layer F.Cu) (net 14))
 (segment (start 116.793 118.665) (end 115.698 118.665) (width 0.3048) (layer F.Cu) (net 14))
 (segment (start 115.698 120.665) (end 116.952 120.665) (width 0.25) (layer F.Cu) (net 15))
 (segment (start 117.729 120.142) (end 118.491 119.38) (width 0.25) (layer B.Cu) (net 15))
 (segment (start 117.475 120.142) (end 117.729 120.142) (width 0.25) (layer B.Cu) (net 15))
 (via (at 117.475 120.142) (size 0.6) (drill 0.4) (layers F.Cu B.Cu) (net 15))
 (segment (start 116.952 120.665) (end 117.475 120.142) (width 0.25) (layer F.Cu) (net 15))
 (segment (start 115.698 110.665) (end 114.887 110.665) (width 0.25) (layer F.Cu) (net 11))
 (segment (start 114.887 110.665) (end 113.665 111.887) (width 0.25) (layer F.Cu) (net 11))
 (segment (start 116.713 121.285) (end 118.491 121.285) (width 0.25) (layer B.Cu) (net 11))
 (segment (start 113.665 118.237) (end 116.713 121.285) (width 0.25) (layer B.Cu) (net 11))
 (segment (start 113.665 116.205) (end 113.665 118.237) (width 0.25) (layer B.Cu) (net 11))
 (via (at 113.665 116.205) (size 0.6) (drill 0.4) (layers F.Cu B.Cu) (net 11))
 (segment (start 113.665 111.887) (end 113.665 116.205) (width 0.25) (layer F.Cu) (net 11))
 (segment (start 118.491 123.19) (end 118.491 124.079) (width 0.25) (layer B.Cu) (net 9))
 (segment (start 129.841 108.665) (end 131.698 108.665) (width 0.25) (layer F.Cu) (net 9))
 (segment (start 129.794 108.712) (end 129.841 108.665) (width 0.25) (layer F.Cu) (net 9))
 (via (at 129.794 108.712) (size 0.6) (drill 0.4) (layers F.Cu B.Cu) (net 9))
 (segment (start 131.699 110.617) (end 129.794 108.712) (width 0.25) (layer B.Cu) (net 9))
 (segment (start 131.699 118.872) (end 131.699 110.617) (width 0.25) (layer B.Cu) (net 9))
 (segment (start 125.984 124.587) (end 131.699 118.872) (width 0.25) (layer B.Cu) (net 9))
 (segment (start 118.999 124.587) (end 125.984 124.587) (width 0.25) (layer B.Cu) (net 9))
 (segment (start 118.491 124.079) (end 118.999 124.587) (width 0.25) (layer B.Cu) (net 9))
 (segment (start 115.698 112.665) (end 117.332 112.665) (width 0.25) (layer F.Cu) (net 2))
 (segment (start 117.602 112.649) (end 118.491 111.76) (width 0.25) (layer B.Cu) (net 2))
 (segment (start 117.348 112.649) (end 117.602 112.649) (width 0.25) (layer B.Cu) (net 2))
 (via (at 117.348 112.649) (size 0.6) (drill 0.4) (layers F.Cu B.Cu) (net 2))
 (segment (start 117.332 112.665) (end 117.348 112.649) (width 0.25) (layer F.Cu) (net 2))
 (segment (start 115.698 112.665) (end 115.714 112.649) (width 0.25) (layer F.Cu) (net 2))
 (segment (start 115.698 116.665) (end 118.92 116.665) (width 0.25) (layer F.Cu) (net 13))
 (segment (start 120.015 115.57) (end 127.381 115.57) (width 0.25) (layer B.Cu) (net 13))
 (via (at 120.015 115.57) (size 0.6) (drill 0.4) (layers F.Cu B.Cu) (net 13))
 (segment (start 118.92 116.665) (end 120.015 115.57) (width 0.25) (layer F.Cu) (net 13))
 (segment (start 127.381 115.57) (end 127.381 113.665) (width 0.25) (layer B.Cu) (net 13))
 (segment (start 115.698 116.665) (end 114.887 116.665) (width 0.3048) (layer F.Cu) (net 13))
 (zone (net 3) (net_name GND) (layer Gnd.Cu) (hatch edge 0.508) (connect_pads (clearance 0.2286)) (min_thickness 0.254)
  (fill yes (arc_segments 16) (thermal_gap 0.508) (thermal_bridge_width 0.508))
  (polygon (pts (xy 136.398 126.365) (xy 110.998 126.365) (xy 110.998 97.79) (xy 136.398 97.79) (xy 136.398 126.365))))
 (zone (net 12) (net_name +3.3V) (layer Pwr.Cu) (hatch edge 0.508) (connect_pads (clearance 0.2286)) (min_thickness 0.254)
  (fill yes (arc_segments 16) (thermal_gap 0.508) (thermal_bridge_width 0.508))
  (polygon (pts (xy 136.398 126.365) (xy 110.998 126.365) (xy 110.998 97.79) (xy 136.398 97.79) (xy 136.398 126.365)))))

